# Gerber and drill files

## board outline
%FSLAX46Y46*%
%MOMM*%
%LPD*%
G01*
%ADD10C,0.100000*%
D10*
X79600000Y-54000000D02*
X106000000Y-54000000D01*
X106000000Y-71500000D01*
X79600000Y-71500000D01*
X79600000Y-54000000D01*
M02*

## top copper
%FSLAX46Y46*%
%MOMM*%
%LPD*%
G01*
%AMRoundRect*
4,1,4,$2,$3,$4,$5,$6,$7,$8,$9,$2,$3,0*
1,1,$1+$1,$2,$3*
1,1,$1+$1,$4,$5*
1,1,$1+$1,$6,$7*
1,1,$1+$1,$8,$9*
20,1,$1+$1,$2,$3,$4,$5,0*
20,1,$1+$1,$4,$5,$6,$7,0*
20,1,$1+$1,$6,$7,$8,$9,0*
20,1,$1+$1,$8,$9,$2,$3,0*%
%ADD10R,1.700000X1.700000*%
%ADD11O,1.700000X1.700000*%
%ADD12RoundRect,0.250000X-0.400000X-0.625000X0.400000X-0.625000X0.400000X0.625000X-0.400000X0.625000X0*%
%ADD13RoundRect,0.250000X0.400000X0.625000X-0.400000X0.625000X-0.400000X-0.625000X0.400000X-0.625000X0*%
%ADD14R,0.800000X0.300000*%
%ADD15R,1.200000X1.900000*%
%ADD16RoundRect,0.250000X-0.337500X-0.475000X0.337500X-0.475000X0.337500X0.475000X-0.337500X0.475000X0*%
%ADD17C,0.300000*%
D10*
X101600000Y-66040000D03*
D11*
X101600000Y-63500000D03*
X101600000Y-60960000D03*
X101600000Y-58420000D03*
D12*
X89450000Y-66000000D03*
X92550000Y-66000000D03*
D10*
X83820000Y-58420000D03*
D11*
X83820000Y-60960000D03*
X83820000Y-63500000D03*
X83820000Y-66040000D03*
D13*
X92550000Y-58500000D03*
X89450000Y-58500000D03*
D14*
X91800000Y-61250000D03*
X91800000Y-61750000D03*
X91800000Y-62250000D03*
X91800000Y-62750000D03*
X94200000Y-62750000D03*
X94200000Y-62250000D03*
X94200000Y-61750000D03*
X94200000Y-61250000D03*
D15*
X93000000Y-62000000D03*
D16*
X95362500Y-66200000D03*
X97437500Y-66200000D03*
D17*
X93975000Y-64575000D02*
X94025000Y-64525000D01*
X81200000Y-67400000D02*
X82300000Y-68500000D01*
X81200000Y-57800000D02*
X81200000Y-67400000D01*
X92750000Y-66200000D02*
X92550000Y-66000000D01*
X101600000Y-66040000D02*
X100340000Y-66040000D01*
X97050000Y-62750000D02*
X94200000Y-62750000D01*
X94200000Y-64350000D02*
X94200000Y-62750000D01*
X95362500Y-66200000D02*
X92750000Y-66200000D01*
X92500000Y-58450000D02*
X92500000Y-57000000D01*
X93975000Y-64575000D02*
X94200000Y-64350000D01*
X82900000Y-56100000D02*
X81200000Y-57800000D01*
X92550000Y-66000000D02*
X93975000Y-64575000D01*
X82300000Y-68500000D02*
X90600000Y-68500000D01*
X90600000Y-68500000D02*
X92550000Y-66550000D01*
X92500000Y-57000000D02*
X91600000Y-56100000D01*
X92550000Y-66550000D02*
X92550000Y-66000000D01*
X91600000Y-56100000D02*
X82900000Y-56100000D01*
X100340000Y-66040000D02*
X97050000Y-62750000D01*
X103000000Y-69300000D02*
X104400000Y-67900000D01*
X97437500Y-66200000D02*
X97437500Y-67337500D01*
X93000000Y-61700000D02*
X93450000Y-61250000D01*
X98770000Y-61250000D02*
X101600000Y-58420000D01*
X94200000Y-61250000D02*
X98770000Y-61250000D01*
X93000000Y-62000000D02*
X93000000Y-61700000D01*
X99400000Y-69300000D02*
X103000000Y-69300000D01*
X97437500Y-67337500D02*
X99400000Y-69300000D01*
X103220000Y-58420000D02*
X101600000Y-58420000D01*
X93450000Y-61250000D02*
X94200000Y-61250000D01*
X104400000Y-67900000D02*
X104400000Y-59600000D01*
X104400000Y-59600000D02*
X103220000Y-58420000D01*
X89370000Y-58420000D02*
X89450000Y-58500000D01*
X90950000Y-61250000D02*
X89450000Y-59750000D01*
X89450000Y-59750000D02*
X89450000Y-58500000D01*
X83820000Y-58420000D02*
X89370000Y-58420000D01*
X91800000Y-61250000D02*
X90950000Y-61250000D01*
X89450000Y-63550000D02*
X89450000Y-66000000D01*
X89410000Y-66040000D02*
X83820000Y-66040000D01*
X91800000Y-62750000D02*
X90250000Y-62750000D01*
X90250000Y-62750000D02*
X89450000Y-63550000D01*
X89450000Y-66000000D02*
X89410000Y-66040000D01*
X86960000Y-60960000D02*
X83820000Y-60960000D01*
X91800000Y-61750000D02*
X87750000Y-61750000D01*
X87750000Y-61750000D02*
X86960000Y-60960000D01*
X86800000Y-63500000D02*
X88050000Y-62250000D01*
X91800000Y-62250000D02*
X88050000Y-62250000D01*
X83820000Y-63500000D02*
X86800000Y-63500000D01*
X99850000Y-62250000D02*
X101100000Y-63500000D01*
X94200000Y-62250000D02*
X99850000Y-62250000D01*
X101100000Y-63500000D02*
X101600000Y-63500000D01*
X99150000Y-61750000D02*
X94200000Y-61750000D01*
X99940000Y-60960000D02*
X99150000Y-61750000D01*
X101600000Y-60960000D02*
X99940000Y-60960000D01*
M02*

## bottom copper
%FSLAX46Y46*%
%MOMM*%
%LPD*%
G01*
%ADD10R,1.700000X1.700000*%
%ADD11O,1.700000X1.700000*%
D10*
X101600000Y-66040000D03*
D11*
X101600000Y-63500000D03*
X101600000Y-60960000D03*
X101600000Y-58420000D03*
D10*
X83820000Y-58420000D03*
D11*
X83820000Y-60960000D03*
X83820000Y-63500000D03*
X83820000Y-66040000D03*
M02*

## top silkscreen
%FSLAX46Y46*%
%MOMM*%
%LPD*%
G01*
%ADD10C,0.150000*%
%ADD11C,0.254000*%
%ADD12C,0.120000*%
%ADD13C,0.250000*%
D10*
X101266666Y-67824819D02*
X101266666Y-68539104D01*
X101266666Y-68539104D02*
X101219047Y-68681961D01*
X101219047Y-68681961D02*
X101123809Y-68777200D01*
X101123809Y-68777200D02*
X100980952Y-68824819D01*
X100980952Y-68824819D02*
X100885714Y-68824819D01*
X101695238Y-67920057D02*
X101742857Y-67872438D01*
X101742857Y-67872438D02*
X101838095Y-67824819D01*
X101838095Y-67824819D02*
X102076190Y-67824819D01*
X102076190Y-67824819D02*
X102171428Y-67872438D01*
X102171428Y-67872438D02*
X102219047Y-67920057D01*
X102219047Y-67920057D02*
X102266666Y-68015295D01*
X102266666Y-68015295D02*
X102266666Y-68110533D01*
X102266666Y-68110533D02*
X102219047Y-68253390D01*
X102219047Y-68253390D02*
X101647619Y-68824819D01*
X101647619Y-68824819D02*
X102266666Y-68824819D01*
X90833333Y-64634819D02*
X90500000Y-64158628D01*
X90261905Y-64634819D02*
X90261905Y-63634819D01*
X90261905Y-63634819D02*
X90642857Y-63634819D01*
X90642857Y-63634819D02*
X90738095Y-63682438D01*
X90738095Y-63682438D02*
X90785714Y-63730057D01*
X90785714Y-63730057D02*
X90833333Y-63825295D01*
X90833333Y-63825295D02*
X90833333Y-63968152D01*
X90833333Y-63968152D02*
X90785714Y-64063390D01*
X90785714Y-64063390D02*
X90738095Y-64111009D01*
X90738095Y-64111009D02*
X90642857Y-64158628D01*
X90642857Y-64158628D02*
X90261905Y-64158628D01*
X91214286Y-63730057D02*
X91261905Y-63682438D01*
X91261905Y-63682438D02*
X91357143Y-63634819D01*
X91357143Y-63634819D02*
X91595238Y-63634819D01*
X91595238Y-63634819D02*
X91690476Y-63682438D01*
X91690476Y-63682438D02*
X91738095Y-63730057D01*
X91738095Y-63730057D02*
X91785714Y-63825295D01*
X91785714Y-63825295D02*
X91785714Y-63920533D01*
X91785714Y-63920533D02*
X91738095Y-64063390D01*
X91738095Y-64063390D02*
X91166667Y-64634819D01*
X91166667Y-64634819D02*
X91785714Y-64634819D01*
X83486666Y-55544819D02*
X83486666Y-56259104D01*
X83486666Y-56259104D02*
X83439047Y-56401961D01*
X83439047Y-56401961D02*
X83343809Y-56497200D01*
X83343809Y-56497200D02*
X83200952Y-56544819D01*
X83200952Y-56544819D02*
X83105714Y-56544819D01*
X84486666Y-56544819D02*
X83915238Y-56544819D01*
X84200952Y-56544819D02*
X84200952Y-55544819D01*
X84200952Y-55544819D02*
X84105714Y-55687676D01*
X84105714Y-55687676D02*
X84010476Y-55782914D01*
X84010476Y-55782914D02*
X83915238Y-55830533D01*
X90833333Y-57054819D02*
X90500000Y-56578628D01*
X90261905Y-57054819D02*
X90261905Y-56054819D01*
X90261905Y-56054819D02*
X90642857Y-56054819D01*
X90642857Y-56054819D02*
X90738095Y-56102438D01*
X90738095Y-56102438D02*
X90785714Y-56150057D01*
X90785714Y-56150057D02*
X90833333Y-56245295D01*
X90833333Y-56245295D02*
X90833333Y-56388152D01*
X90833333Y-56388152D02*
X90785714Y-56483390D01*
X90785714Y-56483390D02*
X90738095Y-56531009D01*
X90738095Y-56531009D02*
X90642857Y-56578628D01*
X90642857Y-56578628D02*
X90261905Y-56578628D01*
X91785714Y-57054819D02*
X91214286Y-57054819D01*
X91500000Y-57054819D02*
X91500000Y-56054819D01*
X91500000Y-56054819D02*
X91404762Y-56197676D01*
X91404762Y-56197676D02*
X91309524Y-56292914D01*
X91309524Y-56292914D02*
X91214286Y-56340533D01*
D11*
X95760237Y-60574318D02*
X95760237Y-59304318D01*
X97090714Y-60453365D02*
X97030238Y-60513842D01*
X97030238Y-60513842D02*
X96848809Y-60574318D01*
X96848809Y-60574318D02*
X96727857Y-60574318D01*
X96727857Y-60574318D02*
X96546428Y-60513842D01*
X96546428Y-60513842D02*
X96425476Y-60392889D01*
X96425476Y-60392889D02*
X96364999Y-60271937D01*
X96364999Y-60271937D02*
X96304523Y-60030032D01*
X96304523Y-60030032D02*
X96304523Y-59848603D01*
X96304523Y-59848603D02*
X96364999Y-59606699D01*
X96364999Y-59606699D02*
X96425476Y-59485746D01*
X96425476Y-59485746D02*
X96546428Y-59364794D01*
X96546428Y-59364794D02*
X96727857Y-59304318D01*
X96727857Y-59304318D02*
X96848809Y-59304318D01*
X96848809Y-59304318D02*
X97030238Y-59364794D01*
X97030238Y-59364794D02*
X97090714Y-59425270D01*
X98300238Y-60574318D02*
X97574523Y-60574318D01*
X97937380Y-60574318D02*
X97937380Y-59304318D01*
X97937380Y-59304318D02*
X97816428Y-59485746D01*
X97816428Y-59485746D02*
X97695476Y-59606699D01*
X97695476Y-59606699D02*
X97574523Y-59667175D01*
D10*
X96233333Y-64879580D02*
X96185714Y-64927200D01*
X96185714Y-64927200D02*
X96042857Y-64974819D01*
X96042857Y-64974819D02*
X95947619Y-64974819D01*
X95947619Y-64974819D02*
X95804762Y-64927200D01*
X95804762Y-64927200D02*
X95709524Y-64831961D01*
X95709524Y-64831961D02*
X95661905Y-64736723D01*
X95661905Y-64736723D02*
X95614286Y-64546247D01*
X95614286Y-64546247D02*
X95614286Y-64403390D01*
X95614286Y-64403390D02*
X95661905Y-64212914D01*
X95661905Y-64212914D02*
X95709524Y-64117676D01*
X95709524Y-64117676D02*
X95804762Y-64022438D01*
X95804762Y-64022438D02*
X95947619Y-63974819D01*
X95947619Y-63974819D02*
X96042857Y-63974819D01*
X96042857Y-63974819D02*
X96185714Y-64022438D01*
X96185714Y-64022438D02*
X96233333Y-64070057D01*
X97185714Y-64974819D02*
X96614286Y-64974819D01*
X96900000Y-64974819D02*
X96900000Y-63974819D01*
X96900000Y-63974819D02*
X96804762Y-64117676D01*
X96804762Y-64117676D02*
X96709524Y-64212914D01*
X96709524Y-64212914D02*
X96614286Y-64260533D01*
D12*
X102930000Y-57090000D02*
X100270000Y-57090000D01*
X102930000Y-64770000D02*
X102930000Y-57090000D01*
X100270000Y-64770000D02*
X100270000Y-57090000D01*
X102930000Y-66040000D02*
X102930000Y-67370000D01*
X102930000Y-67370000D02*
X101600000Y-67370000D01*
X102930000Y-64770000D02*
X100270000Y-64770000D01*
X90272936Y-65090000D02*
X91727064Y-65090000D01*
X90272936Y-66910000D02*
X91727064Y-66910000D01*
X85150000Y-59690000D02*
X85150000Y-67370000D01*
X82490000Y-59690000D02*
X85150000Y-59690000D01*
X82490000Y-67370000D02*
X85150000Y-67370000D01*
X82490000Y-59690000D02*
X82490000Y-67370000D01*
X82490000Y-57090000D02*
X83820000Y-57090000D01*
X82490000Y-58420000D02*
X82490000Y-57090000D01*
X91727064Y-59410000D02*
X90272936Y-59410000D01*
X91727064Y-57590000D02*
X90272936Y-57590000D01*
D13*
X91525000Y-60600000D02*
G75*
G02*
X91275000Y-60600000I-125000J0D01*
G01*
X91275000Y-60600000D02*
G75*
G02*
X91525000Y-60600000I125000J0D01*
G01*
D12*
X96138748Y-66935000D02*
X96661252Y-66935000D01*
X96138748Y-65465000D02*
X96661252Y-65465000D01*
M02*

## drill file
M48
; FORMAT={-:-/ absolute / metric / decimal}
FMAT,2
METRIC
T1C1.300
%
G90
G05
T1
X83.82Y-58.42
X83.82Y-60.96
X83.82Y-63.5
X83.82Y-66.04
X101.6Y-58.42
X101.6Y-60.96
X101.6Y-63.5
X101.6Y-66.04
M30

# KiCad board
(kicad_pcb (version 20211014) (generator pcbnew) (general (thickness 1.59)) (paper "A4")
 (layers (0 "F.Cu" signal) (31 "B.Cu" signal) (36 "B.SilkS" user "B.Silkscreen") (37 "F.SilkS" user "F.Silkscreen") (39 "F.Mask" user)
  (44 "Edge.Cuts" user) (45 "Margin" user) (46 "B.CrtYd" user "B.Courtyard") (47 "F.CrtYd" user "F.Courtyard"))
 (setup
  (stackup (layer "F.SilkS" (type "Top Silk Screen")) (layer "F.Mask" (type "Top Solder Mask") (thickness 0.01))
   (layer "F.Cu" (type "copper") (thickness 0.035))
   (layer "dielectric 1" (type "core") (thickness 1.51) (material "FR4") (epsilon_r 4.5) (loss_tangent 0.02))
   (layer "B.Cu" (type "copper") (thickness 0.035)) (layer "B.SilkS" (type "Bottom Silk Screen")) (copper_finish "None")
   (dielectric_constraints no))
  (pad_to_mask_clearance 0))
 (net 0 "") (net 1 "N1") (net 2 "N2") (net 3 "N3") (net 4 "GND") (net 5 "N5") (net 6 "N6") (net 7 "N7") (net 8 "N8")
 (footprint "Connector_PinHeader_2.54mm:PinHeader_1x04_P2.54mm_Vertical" (layer "F.Cu") (at 101.6 66.04 180)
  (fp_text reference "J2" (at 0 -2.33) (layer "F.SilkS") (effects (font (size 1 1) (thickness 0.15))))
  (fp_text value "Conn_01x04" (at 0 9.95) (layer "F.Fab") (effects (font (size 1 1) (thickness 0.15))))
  (fp_line (start -1.33 8.95) (end 1.33 8.95) (layer "F.SilkS") (width 0.12))
  (fp_line (start -1.33 1.27) (end -1.33 8.95) (layer "F.SilkS") (width 0.12))
  (fp_line (start 1.33 1.27) (end 1.33 8.95) (layer "F.SilkS") (width 0.12))
  (fp_line (start -1.33 0) (end -1.33 -1.33) (layer "F.SilkS") (width 0.12))
  (fp_line (start -1.33 -1.33) (end 0 -1.33) (layer "F.SilkS") (width 0.12))
  (fp_line (start -1.33 1.27) (end 1.33 1.27) (layer "F.SilkS") (width 0.12))
  (pad "1" thru_hole rect (at 0 0 180) (size 1.7 1.7) (drill 1.3) (layers *.Cu *.Mask) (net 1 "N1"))
  (pad "2" thru_hole oval (at 0 2.54 180) (size 1.7 1.7) (drill 1.3) (layers *.Cu *.Mask) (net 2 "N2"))
  (pad "3" thru_hole oval (at 0 5.08 180) (size 1.7 1.7) (drill 1.3) (layers *.Cu *.Mask) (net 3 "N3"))
  (pad "4" thru_hole oval (at 0 7.62 180) (size 1.7 1.7) (drill 1.3) (layers *.Cu *.Mask) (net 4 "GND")))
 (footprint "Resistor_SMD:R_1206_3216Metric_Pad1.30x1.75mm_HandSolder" (layer "F.Cu") (at 91 66)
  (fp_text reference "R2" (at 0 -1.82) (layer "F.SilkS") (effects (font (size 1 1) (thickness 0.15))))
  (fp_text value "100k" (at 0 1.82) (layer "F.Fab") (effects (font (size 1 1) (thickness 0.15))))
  (fp_line (start -0.727064 -0.91) (end 0.727064 -0.91) (layer "F.SilkS") (width 0.12))
  (fp_line (start -0.727064 0.91) (end 0.727064 0.91) (layer "F.SilkS") (width 0.12))
  (pad "1" smd roundrect (at -1.55 0) (size 1.3 1.75) (layers "F.Cu" "F.Paste" "F.Mask") (roundrect_rratio 0.1923076923) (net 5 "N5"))
  (pad "2" smd roundrect (at 1.55 0) (size 1.3 1.75) (layers "F.Cu" "F.Paste" "F.Mask") (roundrect_rratio 0.1923076923) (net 1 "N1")))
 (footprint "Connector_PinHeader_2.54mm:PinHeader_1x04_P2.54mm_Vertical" (layer "F.Cu") (at 83.82 58.42)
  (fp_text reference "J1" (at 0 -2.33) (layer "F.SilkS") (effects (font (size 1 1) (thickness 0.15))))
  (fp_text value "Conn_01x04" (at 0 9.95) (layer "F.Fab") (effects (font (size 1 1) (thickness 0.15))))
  (fp_line (start 1.33 1.27) (end 1.33 8.95) (layer "F.SilkS") (width 0.12))
  (fp_line (start -1.33 1.27) (end 1.33 1.27) (layer "F.SilkS") (width 0.12))
  (fp_line (start -1.33 8.95) (end 1.33 8.95) (layer "F.SilkS") (width 0.12))
  (fp_line (start -1.33 1.27) (end -1.33 8.95) (layer "F.SilkS") (width 0.12))
  (fp_line (start -1.33 -1.33) (end 0 -1.33) (layer "F.SilkS") (width 0.12))
  (fp_line (start -1.33 0) (end -1.33 -1.33) (layer "F.SilkS") (width 0.12))
  (pad "1" thru_hole rect (at 0 0) (size 1.7 1.7) (drill 1.3) (layers *.Cu *.Mask) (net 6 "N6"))
  (pad "2" thru_hole oval (at 0 2.54) (size 1.7 1.7) (drill 1.3) (layers *.Cu *.Mask) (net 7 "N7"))
  (pad "3" thru_hole oval (at 0 5.08) (size 1.7 1.7) (drill 1.3) (layers *.Cu *.Mask) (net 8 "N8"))
  (pad "4" thru_hole oval (at 0 7.62) (size 1.7 1.7) (drill 1.3) (layers *.Cu *.Mask) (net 5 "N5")))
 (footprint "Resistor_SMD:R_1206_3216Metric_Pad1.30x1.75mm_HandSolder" (layer "F.Cu") (at 91 58.5 180)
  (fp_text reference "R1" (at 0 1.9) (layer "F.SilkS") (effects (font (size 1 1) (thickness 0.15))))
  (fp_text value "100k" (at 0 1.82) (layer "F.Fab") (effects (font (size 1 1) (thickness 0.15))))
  (fp_line (start -0.727064 -0.91) (end 0.727064 -0.91) (layer "F.SilkS") (width 0.12))
  (fp_line (start -0.727064 0.91) (end 0.727064 0.91) (layer "F.SilkS") (width 0.12))
  (pad "1" smd roundrect (at -1.55 0 180) (size 1.3 1.75) (layers "F.Cu" "F.Paste" "F.Mask") (roundrect_rratio 0.1923076923) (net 1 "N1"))
  (pad "2" smd roundrect (at 1.55 0 180) (size 1.3 1.75) (layers "F.Cu" "F.Paste" "F.Mask") (roundrect_rratio 0.1923076923) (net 6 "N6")))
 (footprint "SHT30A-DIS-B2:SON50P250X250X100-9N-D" (layer "F.Cu") (at 93 62)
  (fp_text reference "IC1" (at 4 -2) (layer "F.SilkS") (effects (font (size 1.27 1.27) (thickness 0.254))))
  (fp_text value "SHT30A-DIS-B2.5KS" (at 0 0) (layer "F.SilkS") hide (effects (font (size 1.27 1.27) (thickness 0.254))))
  (fp_circle (center -1.6 -1.4) (end -1.6 -1.275) (layer "F.SilkS") (width 0.25) (fill none))
  (pad "1" smd rect locked (at -1.2 -0.75 90) (size 0.3 0.8) (layers "F.Cu" "F.Paste" "F.Mask") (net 6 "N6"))
  (pad "2" smd rect locked (at -1.2 -0.25 90) (size 0.3 0.8) (layers "F.Cu" "F.Paste" "F.Mask") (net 7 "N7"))
  (pad "3" smd rect locked (at -1.2 0.25 90) (size 0.3 0.8) (layers "F.Cu" "F.Paste" "F.Mask") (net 8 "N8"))
  (pad "4" smd rect locked (at -1.2 0.75 90) (size 0.3 0.8) (layers "F.Cu" "F.Paste" "F.Mask") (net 5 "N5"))
  (pad "5" smd rect locked (at 1.2 0.75 90) (size 0.3 0.8) (layers "F.Cu" "F.Paste" "F.Mask") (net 1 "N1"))
  (pad "6" smd rect locked (at 1.2 0.25 90) (size 0.3 0.8) (layers "F.Cu" "F.Paste" "F.Mask") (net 2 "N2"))
  (pad "7" smd rect locked (at 1.2 -0.25 90) (size 0.3 0.8) (layers "F.Cu" "F.Paste" "F.Mask") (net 3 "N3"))
  (pad "8" smd rect locked (at 1.2 -0.75 90) (size 0.3 0.8) (layers "F.Cu" "F.Paste" "F.Mask") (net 4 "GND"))
  (pad "9" smd rect locked (at 0 0) (size 1.2 1.9) (layers "F.Cu" "F.Paste" "F.Mask") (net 4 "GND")))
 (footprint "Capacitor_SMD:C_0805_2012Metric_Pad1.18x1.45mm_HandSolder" (layer "F.Cu") (at 96.4 66.2)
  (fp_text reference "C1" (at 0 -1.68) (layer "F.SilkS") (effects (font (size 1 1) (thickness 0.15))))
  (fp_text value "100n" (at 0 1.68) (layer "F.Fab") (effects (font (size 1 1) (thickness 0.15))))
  (fp_line (start -0.261252 0.735) (end 0.261252 0.735) (layer "F.SilkS") (width 0.12))
  (fp_line (start -0.261252 -0.735) (end 0.261252 -0.735) (layer "F.SilkS") (width 0.12))
  (pad "1" smd roundrect (at -1.0375 0) (size 1.175 1.45) (layers "F.Cu" "F.Paste" "F.Mask") (roundrect_rratio 0.2127659574) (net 1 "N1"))
  (pad "2" smd roundrect (at 1.0375 0) (size 1.175 1.45) (layers "F.Cu" "F.Paste" "F.Mask") (roundrect_rratio 0.2127659574) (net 4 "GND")))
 (gr_rect (start 79.6 54) (end 106 71.5) (layer "Edge.Cuts") (width 0.1) (fill none))
 (segment (start 93.975 64.575) (end 94.025 64.525) (width 0.3) (layer "F.Cu") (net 1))
 (segment (start 81.2 67.4) (end 82.3 68.5) (width 0.3) (layer "F.Cu") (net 1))
 (segment (start 81.2 57.8) (end 81.2 67.4) (width 0.3) (layer "F.Cu") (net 1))
 (segment (start 92.75 66.2) (end 92.55 66) (width 0.3) (layer "F.Cu") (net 1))
 (segment (start 101.6 66.04) (end 100.34 66.04) (width 0.3) (layer "F.Cu") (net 1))
 (segment (start 97.05 62.75) (end 94.2 62.75) (width 0.3) (layer "F.Cu") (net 1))
 (segment (start 94.2 64.35) (end 94.2 62.75) (width 0.3) (layer "F.Cu") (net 1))
 (segment (start 95.3625 66.2) (end 92.75 66.2) (width 0.3) (layer "F.Cu") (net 1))
 (segment (start 92.5 58.45) (end 92.5 57) (width 0.3) (layer "F.Cu") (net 1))
 (segment (start 93.975 64.575) (end 94.2 64.35) (width 0.3) (layer "F.Cu") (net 1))
 (segment (start 82.9 56.1) (end 81.2 57.8) (width 0.3) (layer "F.Cu") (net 1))
 (segment (start 92.55 66) (end 93.975 64.575) (width 0.3) (layer "F.Cu") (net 1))
 (segment (start 82.3 68.5) (end 90.6 68.5) (width 0.3) (layer "F.Cu") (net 1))
 (segment (start 90.6 68.5) (end 92.55 66.55) (width 0.3) (layer "F.Cu") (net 1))
 (segment (start 92.5 57) (end 91.6 56.1) (width 0.3) (layer "F.Cu") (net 1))
 (segment (start 92.55 66.55) (end 92.55 66) (width 0.3) (layer "F.Cu") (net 1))
 (segment (start 91.6 56.1) (end 82.9 56.1) (width 0.3) (layer "F.Cu") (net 1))
 (segment (start 100.34 66.04) (end 97.05 62.75) (width 0.3) (layer "F.Cu") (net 1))
 (segment (start 103 69.3) (end 104.4 67.9) (width 0.3) (layer "F.Cu") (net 4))
 (segment (start 97.4375 66.2) (end 97.4375 67.3375) (width 0.3) (layer "F.Cu") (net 4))
 (segment (start 93 61.7) (end 93.45 61.25) (width 0.3) (layer "F.Cu") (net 4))
 (segment (start 98.77 61.25) (end 101.6 58.42) (width 0.3) (layer "F.Cu") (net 4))
 (segment (start 94.2 61.25) (end 98.77 61.25) (width 0.3) (layer "F.Cu") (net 4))
 (segment (start 93 62) (end 93 61.7) (width 0.3) (layer "F.Cu") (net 4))
 (segment (start 99.4 69.3) (end 103 69.3) (width 0.3) (layer "F.Cu") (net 4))
 (segment (start 97.4375 67.3375) (end 99.4 69.3) (width 0.3) (layer "F.Cu") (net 4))
 (segment (start 103.22 58.42) (end 101.6 58.42) (width 0.3) (layer "F.Cu") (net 4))
 (segment (start 93.45 61.25) (end 94.2 61.25) (width 0.3) (layer "F.Cu") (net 4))
 (segment (start 104.4 67.9) (end 104.4 59.6) (width 0.3) (layer "F.Cu") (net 4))
 (segment (start 104.4 59.6) (end 103.22 58.42) (width 0.3) (layer "F.Cu") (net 4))
 (segment (start 89.37 58.42) (end 89.45 58.5) (width 0.3) (layer "F.Cu") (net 6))
 (segment (start 90.95 61.25) (end 89.45 59.75) (width 0.3) (layer "F.Cu") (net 6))
 (segment (start 89.45 59.75) (end 89.45 58.5) (width 0.3) (layer "F.Cu") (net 6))
 (segment (start 83.82 58.42) (end 89.37 58.42) (width 0.3) (layer "F.Cu") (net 6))
 (segment (start 91.8 61.25) (end 90.95 61.25) (width 0.3) (layer "F.Cu") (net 6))
 (segment (start 89.45 63.55) (end 89.45 66) (width 0.3) (layer "F.Cu") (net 5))
 (segment (start 89.41 66.04) (end 83.82 66.04) (width 0.3) (layer "F.Cu") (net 5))
 (segment (start 91.8 62.75) (end 90.25 62.75) (width 0.3) (layer "F.Cu") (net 5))
 (segment (start 90.25 62.75) (end 89.45 63.55) (width 0.3) (layer "F.Cu") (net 5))
 (segment (start 89.45 66) (end 89.41 66.04) (width 0.3) (layer "F.Cu") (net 5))
 (segment (start 86.96 60.96) (end 83.82 60.96) (width 0.3) (layer "F.Cu") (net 7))
 (segment (start 91.8 61.75) (end 87.75 61.75) (width 0.3) (layer "F.Cu") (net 7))
 (segment (start 87.75 61.75) (end 86.96 60.96) (width 0.3) (layer "F.Cu") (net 7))
 (segment (start 86.8 63.5) (end 88.05 62.25) (width 0.3) (layer "F.Cu") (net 8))
 (segment (start 91.8 62.25) (end 88.05 62.25) (width 0.3) (layer "F.Cu") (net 8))
 (segment (start 83.82 63.5) (end 86.8 63.5) (width 0.3) (layer "F.Cu") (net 8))
 (segment (start 99.85 62.25) (end 101.1 63.5) (width 0.3) (layer "F.Cu") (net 2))
 (segment (start 94.2 62.25) (end 99.85 62.25) (width 0.3) (layer "F.Cu") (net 2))
 (segment (start 101.1 63.5) (end 101.6 63.5) (width 0.3) (layer "F.Cu") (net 2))
 (segment (start 99.15 61.75) (end 94.2 61.75) (width 0.3) (layer "F.Cu") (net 3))
 (segment (start 99.94 60.96) (end 99.15 61.75) (width 0.3) (layer "F.Cu") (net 3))
 (segment (start 101.6 60.96) (end 99.94 60.96) (width 0.3) (layer "F.Cu") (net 3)))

